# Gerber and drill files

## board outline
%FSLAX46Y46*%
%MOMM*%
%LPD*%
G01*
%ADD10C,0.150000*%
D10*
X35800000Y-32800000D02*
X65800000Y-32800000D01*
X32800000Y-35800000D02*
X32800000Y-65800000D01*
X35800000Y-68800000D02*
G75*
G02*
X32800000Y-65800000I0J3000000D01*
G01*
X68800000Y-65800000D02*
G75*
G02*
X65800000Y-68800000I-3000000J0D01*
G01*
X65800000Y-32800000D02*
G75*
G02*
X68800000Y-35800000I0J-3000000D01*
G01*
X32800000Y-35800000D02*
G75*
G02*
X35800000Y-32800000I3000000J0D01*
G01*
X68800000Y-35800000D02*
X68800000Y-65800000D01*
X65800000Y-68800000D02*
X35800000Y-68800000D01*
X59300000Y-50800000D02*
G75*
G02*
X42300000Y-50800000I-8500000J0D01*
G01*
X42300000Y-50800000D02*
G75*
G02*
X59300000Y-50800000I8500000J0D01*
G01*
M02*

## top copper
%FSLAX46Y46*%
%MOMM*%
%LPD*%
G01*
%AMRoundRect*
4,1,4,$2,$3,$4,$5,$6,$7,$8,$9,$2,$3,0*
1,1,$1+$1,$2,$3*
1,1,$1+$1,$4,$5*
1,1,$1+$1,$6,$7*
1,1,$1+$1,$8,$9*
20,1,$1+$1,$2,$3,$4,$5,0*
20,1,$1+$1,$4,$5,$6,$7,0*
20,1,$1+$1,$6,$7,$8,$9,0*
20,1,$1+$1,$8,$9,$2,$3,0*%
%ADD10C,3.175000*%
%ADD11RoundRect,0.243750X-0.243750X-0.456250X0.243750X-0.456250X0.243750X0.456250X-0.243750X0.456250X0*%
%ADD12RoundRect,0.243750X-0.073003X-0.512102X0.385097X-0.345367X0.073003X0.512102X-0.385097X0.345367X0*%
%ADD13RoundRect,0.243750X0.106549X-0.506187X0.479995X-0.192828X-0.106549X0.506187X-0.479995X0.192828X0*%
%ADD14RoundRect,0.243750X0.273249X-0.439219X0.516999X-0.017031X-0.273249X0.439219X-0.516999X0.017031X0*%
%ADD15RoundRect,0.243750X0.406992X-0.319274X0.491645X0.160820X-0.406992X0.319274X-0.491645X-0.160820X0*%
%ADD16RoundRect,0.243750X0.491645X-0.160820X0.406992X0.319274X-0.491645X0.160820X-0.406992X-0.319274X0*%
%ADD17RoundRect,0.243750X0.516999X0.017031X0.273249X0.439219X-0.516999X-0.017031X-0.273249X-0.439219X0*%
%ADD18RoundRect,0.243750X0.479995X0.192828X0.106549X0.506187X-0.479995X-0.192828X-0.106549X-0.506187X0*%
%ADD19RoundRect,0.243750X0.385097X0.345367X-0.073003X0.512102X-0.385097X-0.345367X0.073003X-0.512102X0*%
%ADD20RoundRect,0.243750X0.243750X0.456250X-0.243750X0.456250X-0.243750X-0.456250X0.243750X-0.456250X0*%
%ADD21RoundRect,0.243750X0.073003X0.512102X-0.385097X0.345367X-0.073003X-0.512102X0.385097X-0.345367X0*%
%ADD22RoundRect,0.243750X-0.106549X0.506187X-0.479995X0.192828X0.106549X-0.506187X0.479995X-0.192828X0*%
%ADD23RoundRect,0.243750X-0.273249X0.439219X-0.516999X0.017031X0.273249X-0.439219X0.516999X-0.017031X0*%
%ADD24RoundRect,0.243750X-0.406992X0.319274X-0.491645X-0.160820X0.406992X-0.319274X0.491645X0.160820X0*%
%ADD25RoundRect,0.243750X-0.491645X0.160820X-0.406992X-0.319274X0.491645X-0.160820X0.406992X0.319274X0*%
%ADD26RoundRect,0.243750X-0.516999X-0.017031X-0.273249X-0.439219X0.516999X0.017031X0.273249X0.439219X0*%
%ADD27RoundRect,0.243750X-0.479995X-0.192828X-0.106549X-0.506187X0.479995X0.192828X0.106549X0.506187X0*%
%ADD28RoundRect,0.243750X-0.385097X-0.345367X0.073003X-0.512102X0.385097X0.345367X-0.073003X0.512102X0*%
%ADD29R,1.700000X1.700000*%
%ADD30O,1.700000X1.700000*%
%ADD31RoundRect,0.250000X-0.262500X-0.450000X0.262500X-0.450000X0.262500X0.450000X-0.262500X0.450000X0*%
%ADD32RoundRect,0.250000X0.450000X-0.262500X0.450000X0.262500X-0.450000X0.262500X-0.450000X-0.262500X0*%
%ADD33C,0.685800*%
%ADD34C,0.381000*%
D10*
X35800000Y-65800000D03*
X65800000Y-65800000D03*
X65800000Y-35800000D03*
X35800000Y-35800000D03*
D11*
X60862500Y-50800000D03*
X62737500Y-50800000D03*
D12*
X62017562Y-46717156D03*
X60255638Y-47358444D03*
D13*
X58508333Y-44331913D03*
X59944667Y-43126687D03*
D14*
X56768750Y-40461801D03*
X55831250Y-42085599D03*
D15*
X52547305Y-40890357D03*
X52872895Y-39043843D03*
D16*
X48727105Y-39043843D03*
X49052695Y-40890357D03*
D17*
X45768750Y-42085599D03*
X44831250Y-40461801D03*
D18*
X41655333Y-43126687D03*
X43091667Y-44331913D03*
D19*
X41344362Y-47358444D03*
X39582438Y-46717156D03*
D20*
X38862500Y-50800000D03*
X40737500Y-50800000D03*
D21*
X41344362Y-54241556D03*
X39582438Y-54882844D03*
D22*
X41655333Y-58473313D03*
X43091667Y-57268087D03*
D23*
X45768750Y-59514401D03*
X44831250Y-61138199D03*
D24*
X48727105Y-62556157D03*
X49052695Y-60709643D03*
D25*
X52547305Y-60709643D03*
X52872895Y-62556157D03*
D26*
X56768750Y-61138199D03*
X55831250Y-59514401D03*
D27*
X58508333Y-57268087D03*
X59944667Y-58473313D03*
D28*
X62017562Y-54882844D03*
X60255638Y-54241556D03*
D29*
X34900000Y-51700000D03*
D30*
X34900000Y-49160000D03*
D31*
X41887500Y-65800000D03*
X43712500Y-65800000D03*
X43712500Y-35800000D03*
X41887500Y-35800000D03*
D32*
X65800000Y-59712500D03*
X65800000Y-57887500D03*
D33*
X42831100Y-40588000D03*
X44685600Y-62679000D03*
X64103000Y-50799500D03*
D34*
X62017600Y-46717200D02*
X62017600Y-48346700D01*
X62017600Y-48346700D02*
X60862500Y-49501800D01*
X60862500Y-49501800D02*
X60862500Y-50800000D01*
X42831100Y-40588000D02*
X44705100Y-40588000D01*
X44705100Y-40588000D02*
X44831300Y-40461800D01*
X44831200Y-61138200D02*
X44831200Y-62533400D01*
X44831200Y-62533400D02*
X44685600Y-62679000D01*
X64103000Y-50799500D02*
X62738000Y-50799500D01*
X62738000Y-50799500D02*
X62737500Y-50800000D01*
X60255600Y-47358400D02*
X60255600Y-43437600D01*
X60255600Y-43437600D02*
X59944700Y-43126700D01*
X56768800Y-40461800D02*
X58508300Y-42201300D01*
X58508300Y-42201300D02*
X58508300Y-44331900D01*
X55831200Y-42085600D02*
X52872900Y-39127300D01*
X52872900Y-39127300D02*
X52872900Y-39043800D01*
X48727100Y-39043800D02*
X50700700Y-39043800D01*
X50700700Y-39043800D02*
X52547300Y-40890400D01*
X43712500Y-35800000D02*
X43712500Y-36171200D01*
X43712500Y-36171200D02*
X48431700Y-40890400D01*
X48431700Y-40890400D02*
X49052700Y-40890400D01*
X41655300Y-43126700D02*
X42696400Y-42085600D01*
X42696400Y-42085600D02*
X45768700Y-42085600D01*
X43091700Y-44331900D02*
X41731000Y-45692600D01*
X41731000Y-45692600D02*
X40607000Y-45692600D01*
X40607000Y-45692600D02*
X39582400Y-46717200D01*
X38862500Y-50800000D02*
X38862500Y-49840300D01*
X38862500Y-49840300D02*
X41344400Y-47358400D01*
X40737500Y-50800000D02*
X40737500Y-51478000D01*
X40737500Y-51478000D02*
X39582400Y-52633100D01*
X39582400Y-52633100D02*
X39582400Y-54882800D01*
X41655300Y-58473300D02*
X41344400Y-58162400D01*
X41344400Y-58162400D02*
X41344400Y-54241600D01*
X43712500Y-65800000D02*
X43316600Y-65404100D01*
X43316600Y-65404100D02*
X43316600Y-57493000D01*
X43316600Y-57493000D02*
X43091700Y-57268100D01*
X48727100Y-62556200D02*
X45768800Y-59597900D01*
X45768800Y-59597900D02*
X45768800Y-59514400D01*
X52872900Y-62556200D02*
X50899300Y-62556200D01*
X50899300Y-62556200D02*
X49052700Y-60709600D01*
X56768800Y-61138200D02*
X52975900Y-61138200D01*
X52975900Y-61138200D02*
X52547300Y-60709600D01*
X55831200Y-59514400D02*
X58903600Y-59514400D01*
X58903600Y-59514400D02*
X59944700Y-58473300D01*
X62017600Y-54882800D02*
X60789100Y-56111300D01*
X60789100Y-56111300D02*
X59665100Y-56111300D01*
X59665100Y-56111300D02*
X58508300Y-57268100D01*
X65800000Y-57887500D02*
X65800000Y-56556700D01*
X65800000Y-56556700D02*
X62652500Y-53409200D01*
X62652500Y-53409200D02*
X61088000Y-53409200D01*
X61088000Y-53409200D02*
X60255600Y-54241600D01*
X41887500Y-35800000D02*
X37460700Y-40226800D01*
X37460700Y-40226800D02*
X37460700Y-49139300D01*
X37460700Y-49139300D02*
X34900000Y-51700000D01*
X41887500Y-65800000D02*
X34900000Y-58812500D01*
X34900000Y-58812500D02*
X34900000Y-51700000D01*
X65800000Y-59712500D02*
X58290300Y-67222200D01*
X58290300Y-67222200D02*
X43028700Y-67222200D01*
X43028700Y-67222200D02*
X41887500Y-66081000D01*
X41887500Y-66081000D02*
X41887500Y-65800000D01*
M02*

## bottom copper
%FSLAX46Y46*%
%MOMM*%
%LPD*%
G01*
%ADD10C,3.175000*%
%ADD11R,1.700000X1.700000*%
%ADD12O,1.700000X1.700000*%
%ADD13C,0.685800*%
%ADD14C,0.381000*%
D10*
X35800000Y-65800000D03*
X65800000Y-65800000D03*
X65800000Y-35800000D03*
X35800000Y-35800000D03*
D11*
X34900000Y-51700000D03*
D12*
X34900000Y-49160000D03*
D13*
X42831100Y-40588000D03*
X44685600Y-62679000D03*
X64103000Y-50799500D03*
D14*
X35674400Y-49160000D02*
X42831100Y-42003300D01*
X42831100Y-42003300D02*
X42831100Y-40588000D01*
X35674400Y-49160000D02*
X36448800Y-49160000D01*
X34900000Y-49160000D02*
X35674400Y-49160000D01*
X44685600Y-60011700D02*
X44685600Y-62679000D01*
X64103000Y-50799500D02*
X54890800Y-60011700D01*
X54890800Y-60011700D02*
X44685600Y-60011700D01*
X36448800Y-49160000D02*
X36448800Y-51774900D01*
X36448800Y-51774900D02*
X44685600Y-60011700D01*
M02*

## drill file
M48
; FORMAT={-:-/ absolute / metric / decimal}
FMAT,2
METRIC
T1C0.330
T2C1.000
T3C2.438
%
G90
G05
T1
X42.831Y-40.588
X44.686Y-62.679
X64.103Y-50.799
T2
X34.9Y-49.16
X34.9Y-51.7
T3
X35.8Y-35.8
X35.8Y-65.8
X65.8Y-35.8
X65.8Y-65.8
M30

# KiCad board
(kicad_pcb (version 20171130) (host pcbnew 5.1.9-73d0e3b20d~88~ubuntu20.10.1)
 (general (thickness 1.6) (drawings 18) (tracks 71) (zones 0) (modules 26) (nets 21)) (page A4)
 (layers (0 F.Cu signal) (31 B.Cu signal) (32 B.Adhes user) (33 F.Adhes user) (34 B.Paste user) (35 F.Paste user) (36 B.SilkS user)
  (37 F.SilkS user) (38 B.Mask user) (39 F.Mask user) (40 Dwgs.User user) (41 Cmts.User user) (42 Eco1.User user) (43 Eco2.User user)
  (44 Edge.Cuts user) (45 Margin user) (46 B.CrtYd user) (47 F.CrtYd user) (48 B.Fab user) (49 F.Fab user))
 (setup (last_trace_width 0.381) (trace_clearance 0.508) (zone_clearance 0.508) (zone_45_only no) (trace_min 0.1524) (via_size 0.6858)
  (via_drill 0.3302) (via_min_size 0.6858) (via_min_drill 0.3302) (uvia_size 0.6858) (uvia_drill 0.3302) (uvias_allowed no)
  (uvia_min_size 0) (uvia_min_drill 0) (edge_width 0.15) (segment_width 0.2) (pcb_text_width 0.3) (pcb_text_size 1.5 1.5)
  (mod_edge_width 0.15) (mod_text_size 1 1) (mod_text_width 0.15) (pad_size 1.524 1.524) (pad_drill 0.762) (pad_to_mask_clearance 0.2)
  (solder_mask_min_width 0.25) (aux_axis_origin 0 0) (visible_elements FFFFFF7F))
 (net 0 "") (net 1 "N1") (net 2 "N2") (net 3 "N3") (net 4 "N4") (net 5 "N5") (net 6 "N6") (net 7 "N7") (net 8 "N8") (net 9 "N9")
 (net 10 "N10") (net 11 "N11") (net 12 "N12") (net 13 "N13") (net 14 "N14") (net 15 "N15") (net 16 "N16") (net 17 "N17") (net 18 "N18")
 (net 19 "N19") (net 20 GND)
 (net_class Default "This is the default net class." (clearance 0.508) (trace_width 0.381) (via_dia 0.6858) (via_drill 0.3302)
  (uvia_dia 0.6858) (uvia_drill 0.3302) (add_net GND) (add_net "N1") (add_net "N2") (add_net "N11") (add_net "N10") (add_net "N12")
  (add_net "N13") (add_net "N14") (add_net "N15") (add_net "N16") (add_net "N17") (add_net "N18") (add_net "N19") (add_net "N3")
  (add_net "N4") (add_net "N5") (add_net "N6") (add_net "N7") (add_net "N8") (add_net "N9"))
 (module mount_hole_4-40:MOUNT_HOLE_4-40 (layer F.Cu) (at 35.8 65.8)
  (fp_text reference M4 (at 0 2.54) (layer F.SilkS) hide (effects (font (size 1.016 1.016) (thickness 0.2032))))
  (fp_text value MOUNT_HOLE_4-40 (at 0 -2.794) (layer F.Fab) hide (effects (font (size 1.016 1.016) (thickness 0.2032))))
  (pad 1 thru_hole circle (at 0 0) (size 3.175 3.175) (drill 2.4384) (layers *.Cu *.Mask)))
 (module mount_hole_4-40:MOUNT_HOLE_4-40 (layer F.Cu) (at 65.8 65.8)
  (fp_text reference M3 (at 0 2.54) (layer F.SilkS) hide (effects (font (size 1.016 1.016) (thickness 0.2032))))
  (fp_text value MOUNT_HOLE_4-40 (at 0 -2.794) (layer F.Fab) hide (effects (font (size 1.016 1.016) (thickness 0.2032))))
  (pad 1 thru_hole circle (at 0 0) (size 3.175 3.175) (drill 2.4384) (layers *.Cu *.Mask)))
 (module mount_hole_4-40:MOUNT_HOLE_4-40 (layer F.Cu) (at 65.8 35.8)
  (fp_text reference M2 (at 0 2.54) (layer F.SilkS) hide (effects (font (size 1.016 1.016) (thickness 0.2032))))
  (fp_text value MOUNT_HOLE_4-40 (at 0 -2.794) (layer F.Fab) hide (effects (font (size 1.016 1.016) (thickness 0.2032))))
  (pad 1 thru_hole circle (at 0 0) (size 3.175 3.175) (drill 2.4384) (layers *.Cu *.Mask)))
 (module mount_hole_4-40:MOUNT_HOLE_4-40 (layer F.Cu) (at 35.8 35.8)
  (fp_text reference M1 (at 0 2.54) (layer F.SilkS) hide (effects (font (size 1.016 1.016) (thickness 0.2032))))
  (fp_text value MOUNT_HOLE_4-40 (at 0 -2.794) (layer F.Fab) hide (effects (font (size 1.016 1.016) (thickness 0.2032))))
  (pad 1 thru_hole circle (at 0 0) (size 3.175 3.175) (drill 2.4384) (layers *.Cu *.Mask)))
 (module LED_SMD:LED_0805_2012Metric (layer F.Cu) (at 61.8 50.8)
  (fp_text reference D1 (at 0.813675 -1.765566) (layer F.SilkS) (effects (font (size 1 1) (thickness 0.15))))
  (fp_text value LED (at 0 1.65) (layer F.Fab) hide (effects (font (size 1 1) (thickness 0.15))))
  (pad 1 smd roundrect (at -0.9375 0) (size 0.975 1.4) (layers F.Cu F.Paste F.Mask) (roundrect_rratio 0.25) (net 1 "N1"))
  (pad 2 smd roundrect (at 0.9375 0) (size 0.975 1.4) (layers F.Cu F.Paste F.Mask) (roundrect_rratio 0.25) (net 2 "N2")))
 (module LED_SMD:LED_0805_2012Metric (layer F.Cu) (at 61.1366 47.0378 20)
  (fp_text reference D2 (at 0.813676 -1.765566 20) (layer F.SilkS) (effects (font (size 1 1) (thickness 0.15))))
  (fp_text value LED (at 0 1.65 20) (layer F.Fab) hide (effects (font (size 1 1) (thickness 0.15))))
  (pad 2 smd roundrect (at 0.9375 0 20) (size 0.975 1.4) (layers F.Cu F.Paste F.Mask) (roundrect_rratio 0.25) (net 1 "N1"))
  (pad 1 smd roundrect (at -0.9375 0 20) (size 0.975 1.4) (layers F.Cu F.Paste F.Mask) (roundrect_rratio 0.25) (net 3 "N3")))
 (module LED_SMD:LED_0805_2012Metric (layer F.Cu) (at 59.2265 43.7293 40)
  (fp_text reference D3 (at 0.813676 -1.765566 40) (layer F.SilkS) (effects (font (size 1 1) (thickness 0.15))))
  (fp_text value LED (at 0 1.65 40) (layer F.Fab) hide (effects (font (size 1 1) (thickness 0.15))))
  (pad 1 smd roundrect (at -0.9375 0 40) (size 0.975 1.4) (layers F.Cu F.Paste F.Mask) (roundrect_rratio 0.25) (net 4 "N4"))
  (pad 2 smd roundrect (at 0.9375 0 40) (size 0.975 1.4) (layers F.Cu F.Paste F.Mask) (roundrect_rratio 0.25) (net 3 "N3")))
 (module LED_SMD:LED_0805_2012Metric (layer F.Cu) (at 56.3 41.2737 60)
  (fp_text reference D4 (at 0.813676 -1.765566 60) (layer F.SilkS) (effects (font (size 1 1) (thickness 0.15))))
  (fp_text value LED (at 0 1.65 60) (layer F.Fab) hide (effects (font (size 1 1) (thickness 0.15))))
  (pad 2 smd roundrect (at 0.9375 0 60) (size 0.975 1.4) (layers F.Cu F.Paste F.Mask) (roundrect_rratio 0.25) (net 4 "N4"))
  (pad 1 smd roundrect (at -0.9375 0 60) (size 0.975 1.4) (layers F.Cu F.Paste F.Mask) (roundrect_rratio 0.25) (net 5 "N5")))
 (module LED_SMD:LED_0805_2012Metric (layer F.Cu) (at 52.7101 39.9671 80)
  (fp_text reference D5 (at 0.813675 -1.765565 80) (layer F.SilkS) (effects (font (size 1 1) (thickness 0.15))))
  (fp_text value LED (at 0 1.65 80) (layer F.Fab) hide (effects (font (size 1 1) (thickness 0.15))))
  (pad 1 smd roundrect (at -0.9375 0 80) (size 0.975 1.4) (layers F.Cu F.Paste F.Mask) (roundrect_rratio 0.25) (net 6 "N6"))
  (pad 2 smd roundrect (at 0.9375 0 80) (size 0.975 1.4) (layers F.Cu F.Paste F.Mask) (roundrect_rratio 0.25) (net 5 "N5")))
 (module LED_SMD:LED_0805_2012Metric (layer F.Cu) (at 48.8899 39.9671 100)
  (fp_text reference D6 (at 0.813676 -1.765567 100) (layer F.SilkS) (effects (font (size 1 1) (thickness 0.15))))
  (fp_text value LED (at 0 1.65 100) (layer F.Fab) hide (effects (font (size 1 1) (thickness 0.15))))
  (pad 2 smd roundrect (at 0.9375 0 100) (size 0.975 1.4) (layers F.Cu F.Paste F.Mask) (roundrect_rratio 0.25) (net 6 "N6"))
  (pad 1 smd roundrect (at -0.9375 0 100) (size 0.975 1.4) (layers F.Cu F.Paste F.Mask) (roundrect_rratio 0.25) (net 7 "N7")))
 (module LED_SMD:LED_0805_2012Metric (layer F.Cu) (at 45.3 41.2737 120)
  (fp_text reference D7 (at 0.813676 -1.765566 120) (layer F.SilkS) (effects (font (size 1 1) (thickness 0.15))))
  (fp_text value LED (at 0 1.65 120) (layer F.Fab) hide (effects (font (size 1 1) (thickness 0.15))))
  (pad 1 smd roundrect (at -0.9375 0 120) (size 0.975 1.4) (layers F.Cu F.Paste F.Mask) (roundrect_rratio 0.25) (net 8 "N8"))
  (pad 2 smd roundrect (at 0.9375 0 120) (size 0.975 1.4) (layers F.Cu F.Paste F.Mask) (roundrect_rratio 0.25) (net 2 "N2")))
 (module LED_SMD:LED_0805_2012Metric (layer F.Cu) (at 42.3735 43.7293 140)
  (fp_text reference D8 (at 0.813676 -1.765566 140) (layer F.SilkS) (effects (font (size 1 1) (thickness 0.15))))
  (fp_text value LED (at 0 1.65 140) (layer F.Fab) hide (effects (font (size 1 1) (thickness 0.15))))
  (pad 2 smd roundrect (at 0.9375 0 140) (size 0.975 1.4) (layers F.Cu F.Paste F.Mask) (roundrect_rratio 0.25) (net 8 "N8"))
  (pad 1 smd roundrect (at -0.9375 0 140) (size 0.975 1.4) (layers F.Cu F.Paste F.Mask) (roundrect_rratio 0.25) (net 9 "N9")))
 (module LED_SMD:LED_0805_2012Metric (layer F.Cu) (at 40.4634 47.0378 160)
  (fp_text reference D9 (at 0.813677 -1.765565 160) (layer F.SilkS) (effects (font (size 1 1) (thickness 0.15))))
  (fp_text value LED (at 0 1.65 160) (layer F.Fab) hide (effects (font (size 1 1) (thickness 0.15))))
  (pad 1 smd roundrect (at -0.9375 0 160) (size 0.975 1.4) (layers F.Cu F.Paste F.Mask) (roundrect_rratio 0.25) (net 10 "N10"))
  (pad 2 smd roundrect (at 0.9375 0 160) (size 0.975 1.4) (layers F.Cu F.Paste F.Mask) (roundrect_rratio 0.25) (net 9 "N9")))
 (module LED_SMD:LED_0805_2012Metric (layer F.Cu) (at 39.8 50.8 180)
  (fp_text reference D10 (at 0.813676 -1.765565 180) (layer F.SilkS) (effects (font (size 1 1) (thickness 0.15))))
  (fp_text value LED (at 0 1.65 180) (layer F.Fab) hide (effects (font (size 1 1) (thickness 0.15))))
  (pad 2 smd roundrect (at 0.9375 0 180) (size 0.975 1.4) (layers F.Cu F.Paste F.Mask) (roundrect_rratio 0.25) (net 10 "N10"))
  (pad 1 smd roundrect (at -0.9375 0 180) (size 0.975 1.4) (layers F.Cu F.Paste F.Mask) (roundrect_rratio 0.25) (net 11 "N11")))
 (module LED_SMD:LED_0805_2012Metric (layer F.Cu) (at 40.4634 54.5622 200)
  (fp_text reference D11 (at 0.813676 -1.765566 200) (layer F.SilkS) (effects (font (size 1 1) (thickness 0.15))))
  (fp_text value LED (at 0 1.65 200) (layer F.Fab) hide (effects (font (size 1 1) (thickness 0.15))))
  (pad 1 smd roundrect (at -0.9375 0 200) (size 0.975 1.4) (layers F.Cu F.Paste F.Mask) (roundrect_rratio 0.25) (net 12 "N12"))
  (pad 2 smd roundrect (at 0.9375 0 200) (size 0.975 1.4) (layers F.Cu F.Paste F.Mask) (roundrect_rratio 0.25) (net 11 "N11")))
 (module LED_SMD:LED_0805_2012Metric (layer F.Cu) (at 42.3735 57.8707 220)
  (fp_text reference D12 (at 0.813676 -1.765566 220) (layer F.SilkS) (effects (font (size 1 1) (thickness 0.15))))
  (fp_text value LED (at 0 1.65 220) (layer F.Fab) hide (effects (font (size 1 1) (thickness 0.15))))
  (pad 2 smd roundrect (at 0.9375 0 220) (size 0.975 1.4) (layers F.Cu F.Paste F.Mask) (roundrect_rratio 0.25) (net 12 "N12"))
  (pad 1 smd roundrect (at -0.9375 0 220) (size 0.975 1.4) (layers F.Cu F.Paste F.Mask) (roundrect_rratio 0.25) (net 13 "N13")))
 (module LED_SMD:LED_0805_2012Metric (layer F.Cu) (at 45.3 60.3263 240)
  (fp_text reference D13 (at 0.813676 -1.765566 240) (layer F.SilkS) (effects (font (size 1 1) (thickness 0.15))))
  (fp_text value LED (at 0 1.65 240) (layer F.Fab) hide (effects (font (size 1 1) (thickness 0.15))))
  (pad 1 smd roundrect (at -0.9375 0 240) (size 0.975 1.4) (layers F.Cu F.Paste F.Mask) (roundrect_rratio 0.25) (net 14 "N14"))
  (pad 2 smd roundrect (at 0.9375 0 240) (size 0.975 1.4) (layers F.Cu F.Paste F.Mask) (roundrect_rratio 0.25) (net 2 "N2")))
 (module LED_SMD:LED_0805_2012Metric (layer F.Cu) (at 48.8899 61.6329 260)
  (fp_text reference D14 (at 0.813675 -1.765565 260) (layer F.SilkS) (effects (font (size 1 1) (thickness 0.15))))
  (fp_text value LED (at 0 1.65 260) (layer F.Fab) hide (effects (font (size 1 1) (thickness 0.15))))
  (pad 2 smd roundrect (at 0.9375 0 260) (size 0.975 1.4) (layers F.Cu F.Paste F.Mask) (roundrect_rratio 0.25) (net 14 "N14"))
  (pad 1 smd roundrect (at -0.9375 0 260) (size 0.975 1.4) (layers F.Cu F.Paste F.Mask) (roundrect_rratio 0.25) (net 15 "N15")))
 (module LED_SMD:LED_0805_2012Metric (layer F.Cu) (at 52.7101 61.6329 280)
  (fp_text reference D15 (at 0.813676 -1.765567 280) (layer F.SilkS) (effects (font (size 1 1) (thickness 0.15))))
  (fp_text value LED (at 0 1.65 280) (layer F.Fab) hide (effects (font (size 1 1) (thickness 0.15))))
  (pad 1 smd roundrect (at -0.9375 0 280) (size 0.975 1.4) (layers F.Cu F.Paste F.Mask) (roundrect_rratio 0.25) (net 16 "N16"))
  (pad 2 smd roundrect (at 0.9375 0 280) (size 0.975 1.4) (layers F.Cu F.Paste F.Mask) (roundrect_rratio 0.25) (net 15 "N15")))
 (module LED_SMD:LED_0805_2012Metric (layer F.Cu) (at 56.3 60.3263 300)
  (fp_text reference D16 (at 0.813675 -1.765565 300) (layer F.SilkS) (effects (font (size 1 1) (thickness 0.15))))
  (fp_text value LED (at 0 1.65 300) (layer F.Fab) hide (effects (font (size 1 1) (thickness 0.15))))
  (pad 2 smd roundrect (at 0.9375 0 300) (size 0.975 1.4) (layers F.Cu F.Paste F.Mask) (roundrect_rratio 0.25) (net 16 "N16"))
  (pad 1 smd roundrect (at -0.9375 0 300) (size 0.975 1.4) (layers F.Cu F.Paste F.Mask) (roundrect_rratio 0.25) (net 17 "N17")))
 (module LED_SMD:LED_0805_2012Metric (layer F.Cu) (at 59.2265 57.8707 320)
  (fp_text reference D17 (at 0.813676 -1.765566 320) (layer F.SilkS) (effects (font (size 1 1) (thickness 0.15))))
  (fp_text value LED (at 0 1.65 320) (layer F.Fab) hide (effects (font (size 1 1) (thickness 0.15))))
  (pad 1 smd roundrect (at -0.9375 0 320) (size 0.975 1.4) (layers F.Cu F.Paste F.Mask) (roundrect_rratio 0.25) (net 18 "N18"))
  (pad 2 smd roundrect (at 0.9375 0 320) (size 0.975 1.4) (layers F.Cu F.Paste F.Mask) (roundrect_rratio 0.25) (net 17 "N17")))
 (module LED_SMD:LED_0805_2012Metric (layer F.Cu) (at 61.1366 54.5622 340)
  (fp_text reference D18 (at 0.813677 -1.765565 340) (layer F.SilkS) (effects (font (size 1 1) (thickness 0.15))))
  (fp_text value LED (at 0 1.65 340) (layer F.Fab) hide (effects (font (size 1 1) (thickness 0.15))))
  (pad 2 smd roundrect (at 0.9375 0 340) (size 0.975 1.4) (layers F.Cu F.Paste F.Mask) (roundrect_rratio 0.25) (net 18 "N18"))
  (pad 1 smd roundrect (at -0.9375 0 340) (size 0.975 1.4) (layers F.Cu F.Paste F.Mask) (roundrect_rratio 0.25) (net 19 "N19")))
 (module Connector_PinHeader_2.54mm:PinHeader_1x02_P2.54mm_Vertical (layer B.Cu) (at 34.9 51.7)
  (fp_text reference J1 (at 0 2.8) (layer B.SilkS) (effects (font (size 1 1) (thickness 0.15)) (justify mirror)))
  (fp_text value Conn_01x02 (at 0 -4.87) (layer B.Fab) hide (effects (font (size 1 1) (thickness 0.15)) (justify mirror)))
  (pad 1 thru_hole rect (at 0 0) (size 1.7 1.7) (drill 1) (layers *.Cu *.Mask) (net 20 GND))
  (pad 2 thru_hole oval (at 0 -2.54) (size 1.7 1.7) (drill 1) (layers *.Cu *.Mask) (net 2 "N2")))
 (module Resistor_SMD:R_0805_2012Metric (layer F.Cu) (at 42.8 65.8)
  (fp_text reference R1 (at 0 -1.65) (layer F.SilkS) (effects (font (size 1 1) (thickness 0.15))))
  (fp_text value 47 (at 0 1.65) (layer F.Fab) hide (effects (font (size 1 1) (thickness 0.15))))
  (pad 1 smd roundrect (at -0.9125 0) (size 1.025 1.4) (layers F.Cu F.Paste F.Mask) (roundrect_rratio 0.243902) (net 20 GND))
  (pad 2 smd roundrect (at 0.9125 0) (size 1.025 1.4) (layers F.Cu F.Paste F.Mask) (roundrect_rratio 0.243902) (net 13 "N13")))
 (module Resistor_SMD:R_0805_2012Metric (layer F.Cu) (at 42.8 35.8)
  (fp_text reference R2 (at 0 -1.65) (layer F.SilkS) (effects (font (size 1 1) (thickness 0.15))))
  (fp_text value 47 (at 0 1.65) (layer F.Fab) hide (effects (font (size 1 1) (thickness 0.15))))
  (pad 2 smd roundrect (at 0.9125 0) (size 1.025 1.4) (layers F.Cu F.Paste F.Mask) (roundrect_rratio 0.243902) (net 7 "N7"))
  (pad 1 smd roundrect (at -0.9125 0) (size 1.025 1.4) (layers F.Cu F.Paste F.Mask) (roundrect_rratio 0.243902) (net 20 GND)))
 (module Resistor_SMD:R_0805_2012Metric (layer F.Cu) (at 65.8 58.8 90)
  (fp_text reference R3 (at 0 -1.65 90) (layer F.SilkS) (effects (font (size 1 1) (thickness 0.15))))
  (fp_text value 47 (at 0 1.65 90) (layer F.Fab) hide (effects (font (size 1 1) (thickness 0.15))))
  (pad 1 smd roundrect (at -0.9125 0 90) (size 1.025 1.4) (layers F.Cu F.Paste F.Mask) (roundrect_rratio 0.243902) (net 20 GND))
  (pad 2 smd roundrect (at 0.9125 0 90) (size 1.025 1.4) (layers F.Cu F.Paste F.Mask) (roundrect_rratio 0.243902) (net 19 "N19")))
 (gr_line (start 35.8 32.8) (end 65.8 32.8) (layer Edge.Cuts) (width 0.15))
 (gr_line (start 32.8 35.8) (end 32.8 65.8) (layer Edge.Cuts) (width 0.15))
 (gr_arc (start 35.8 65.8) (end 32.8 65.8) (angle -90) (layer Edge.Cuts) (width 0.15))
 (gr_arc (start 65.8 65.8) (end 65.8 68.8) (angle -90) (layer Edge.Cuts) (width 0.15))
 (gr_arc (start 65.8 35.8) (end 68.8 35.8) (angle -90) (layer Edge.Cuts) (width 0.15))
 (gr_arc (start 35.8 35.8) (end 35.8 32.8) (angle -90) (layer Edge.Cuts) (width 0.15))
 (gr_line (start 68.8 35.8) (end 68.8 65.8) (layer Edge.Cuts) (width 0.15))
 (gr_line (start 65.8 68.8) (end 35.8 68.8) (layer Edge.Cuts) (width 0.15))
 (gr_circle (center 50.8 50.8) (end 59.3 50.8) (layer Edge.Cuts) (width 0.15))
 (segment (start 62.0176 46.7172) (end 62.0176 48.3467) (width 0.381) (layer F.Cu) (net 1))
 (segment (start 62.0176 48.3467) (end 60.8625 49.5018) (width 0.381) (layer F.Cu) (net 1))
 (segment (start 60.8625 49.5018) (end 60.8625 50.8) (width 0.381) (layer F.Cu) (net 1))
 (segment (start 42.8311 40.588) (end 44.7051 40.588) (width 0.381) (layer F.Cu) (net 2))
 (segment (start 44.7051 40.588) (end 44.8313 40.4618) (width 0.381) (layer F.Cu) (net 2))
 (segment (start 35.6744 49.16) (end 42.8311 42.0033) (width 0.381) (layer B.Cu) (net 2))
 (segment (start 42.8311 42.0033) (end 42.8311 40.588) (width 0.381) (layer B.Cu) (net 2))
 (segment (start 35.6744 49.16) (end 36.4488 49.16) (width 0.381) (layer B.Cu) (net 2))
 (segment (start 34.9 49.16) (end 35.6744 49.16) (width 0.381) (layer B.Cu) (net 2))
 (segment (start 44.6856 60.0117) (end 44.6856 62.679) (width 0.381) (layer B.Cu) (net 2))
 (segment (start 64.103 50.7995) (end 54.8908 60.0117) (width 0.381) (layer B.Cu) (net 2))
 (segment (start 54.8908 60.0117) (end 44.6856 60.0117) (width 0.381) (layer B.Cu) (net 2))
 (segment (start 36.4488 49.16) (end 36.4488 51.7749) (width 0.381) (layer B.Cu) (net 2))
 (segment (start 36.4488 51.7749) (end 44.6856 60.0117) (width 0.381) (layer B.Cu) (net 2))
 (segment (start 44.8312 61.1382) (end 44.8312 62.5334) (width 0.381) (layer F.Cu) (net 2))
 (segment (start 44.8312 62.5334) (end 44.6856 62.679) (width 0.381) (layer F.Cu) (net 2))
 (segment (start 64.103 50.7995) (end 62.738 50.7995) (width 0.381) (layer F.Cu) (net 2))
 (segment (start 62.738 50.7995) (end 62.7375 50.8) (width 0.381) (layer F.Cu) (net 2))
 (via (at 42.8311 40.588) (size 0.6858) (layers F.Cu B.Cu) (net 2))
 (via (at 44.6856 62.679) (size 0.6858) (layers F.Cu B.Cu) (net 2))
 (via (at 64.103 50.7995) (size 0.6858) (layers F.Cu B.Cu) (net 2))
 (segment (start 60.2556 47.3584) (end 60.2556 43.4376) (width 0.381) (layer F.Cu) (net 3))
 (segment (start 60.2556 43.4376) (end 59.9447 43.1267) (width 0.381) (layer F.Cu) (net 3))
 (segment (start 56.7688 40.4618) (end 58.5083 42.2013) (width 0.381) (layer F.Cu) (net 4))
 (segment (start 58.5083 42.2013) (end 58.5083 44.3319) (width 0.381) (layer F.Cu) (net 4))
 (segment (start 55.8312 42.0856) (end 52.8729 39.1273) (width 0.381) (layer F.Cu) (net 5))
 (segment (start 52.8729 39.1273) (end 52.8729 39.0438) (width 0.381) (layer F.Cu) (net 5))
 (segment (start 48.7271 39.0438) (end 50.7007 39.0438) (width 0.381) (layer F.Cu) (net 6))
 (segment (start 50.7007 39.0438) (end 52.5473 40.8904) (width 0.381) (layer F.Cu) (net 6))
 (segment (start 43.7125 35.8) (end 43.7125 36.1712) (width 0.381) (layer F.Cu) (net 7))
 (segment (start 43.7125 36.1712) (end 48.4317 40.8904) (width 0.381) (layer F.Cu) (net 7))
 (segment (start 48.4317 40.8904) (end 49.0527 40.8904) (width 0.381) (layer F.Cu) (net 7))
 (segment (start 41.6553 43.1267) (end 42.6964 42.0856) (width 0.381) (layer F.Cu) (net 8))
 (segment (start 42.6964 42.0856) (end 45.7687 42.0856) (width 0.381) (layer F.Cu) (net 8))
 (segment (start 43.0917 44.3319) (end 41.731 45.6926) (width 0.381) (layer F.Cu) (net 9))
 (segment (start 41.731 45.6926) (end 40.607 45.6926) (width 0.381) (layer F.Cu) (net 9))
 (segment (start 40.607 45.6926) (end 39.5824 46.7172) (width 0.381) (layer F.Cu) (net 9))
 (segment (start 38.8625 50.8) (end 38.8625 49.8403) (width 0.381) (layer F.Cu) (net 10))
 (segment (start 38.8625 49.8403) (end 41.3444 47.3584) (width 0.381) (layer F.Cu) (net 10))
 (segment (start 40.7375 50.8) (end 40.7375 51.478) (width 0.381) (layer F.Cu) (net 11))
 (segment (start 40.7375 51.478) (end 39.5824 52.6331) (width 0.381) (layer F.Cu) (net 11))
 (segment (start 39.5824 52.6331) (end 39.5824 54.8828) (width 0.381) (layer F.Cu) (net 11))
 (segment (start 41.6553 58.4733) (end 41.3444 58.1624) (width 0.381) (layer F.Cu) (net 12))
 (segment (start 41.3444 58.1624) (end 41.3444 54.2416) (width 0.381) (layer F.Cu) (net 12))
 (segment (start 43.7125 65.8) (end 43.3166 65.4041) (width 0.381) (layer F.Cu) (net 13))
 (segment (start 43.3166 65.4041) (end 43.3166 57.493) (width 0.381) (layer F.Cu) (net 13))
 (segment (start 43.3166 57.493) (end 43.0917 57.2681) (width 0.381) (layer F.Cu) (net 13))
 (segment (start 48.7271 62.5562) (end 45.7688 59.5979) (width 0.381) (layer F.Cu) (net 14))
 (segment (start 45.7688 59.5979) (end 45.7688 59.5144) (width 0.381) (layer F.Cu) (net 14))
 (segment (start 52.8729 62.5562) (end 50.8993 62.5562) (width 0.381) (layer F.Cu) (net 15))
 (segment (start 50.8993 62.5562) (end 49.0527 60.7096) (width 0.381) (layer F.Cu) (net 15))
 (segment (start 56.7688 61.1382) (end 52.9759 61.1382) (width 0.381) (layer F.Cu) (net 16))
 (segment (start 52.9759 61.1382) (end 52.5473 60.7096) (width 0.381) (layer F.Cu) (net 16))
 (segment (start 55.8312 59.5144) (end 58.9036 59.5144) (width 0.381) (layer F.Cu) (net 17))
 (segment (start 58.9036 59.5144) (end 59.9447 58.4733) (width 0.381) (layer F.Cu) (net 17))
 (segment (start 62.0176 54.8828) (end 60.7891 56.1113) (width 0.381) (layer F.Cu) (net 18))
 (segment (start 60.7891 56.1113) (end 59.6651 56.1113) (width 0.381) (layer F.Cu) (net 18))
 (segment (start 59.6651 56.1113) (end 58.5083 57.2681) (width 0.381) (layer F.Cu) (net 18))
 (segment (start 65.8 57.8875) (end 65.8 56.5567) (width 0.381) (layer F.Cu) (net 19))
 (segment (start 65.8 56.5567) (end 62.6525 53.4092) (width 0.381) (layer F.Cu) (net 19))
 (segment (start 62.6525 53.4092) (end 61.088 53.4092) (width 0.381) (layer F.Cu) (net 19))
 (segment (start 61.088 53.4092) (end 60.2556 54.2416) (width 0.381) (layer F.Cu) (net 19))
 (segment (start 41.8875 35.8) (end 37.4607 40.2268) (width 0.381) (layer F.Cu) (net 20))
 (segment (start 37.4607 40.2268) (end 37.4607 49.1393) (width 0.381) (layer F.Cu) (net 20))
 (segment (start 37.4607 49.1393) (end 34.9 51.7) (width 0.381) (layer F.Cu) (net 20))
 (segment (start 41.8875 65.8) (end 34.9 58.8125) (width 0.381) (layer F.Cu) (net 20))
 (segment (start 34.9 58.8125) (end 34.9 51.7) (width 0.381) (layer F.Cu) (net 20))
 (segment (start 65.8 59.7125) (end 58.2903 67.2222) (width 0.381) (layer F.Cu) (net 20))
 (segment (start 58.2903 67.2222) (end 43.0287 67.2222) (width 0.381) (layer F.Cu) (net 20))
 (segment (start 43.0287 67.2222) (end 41.8875 66.081) (width 0.381) (layer F.Cu) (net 20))
 (segment (start 41.8875 66.081) (end 41.8875 65.8) (width 0.381) (layer F.Cu) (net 20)))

